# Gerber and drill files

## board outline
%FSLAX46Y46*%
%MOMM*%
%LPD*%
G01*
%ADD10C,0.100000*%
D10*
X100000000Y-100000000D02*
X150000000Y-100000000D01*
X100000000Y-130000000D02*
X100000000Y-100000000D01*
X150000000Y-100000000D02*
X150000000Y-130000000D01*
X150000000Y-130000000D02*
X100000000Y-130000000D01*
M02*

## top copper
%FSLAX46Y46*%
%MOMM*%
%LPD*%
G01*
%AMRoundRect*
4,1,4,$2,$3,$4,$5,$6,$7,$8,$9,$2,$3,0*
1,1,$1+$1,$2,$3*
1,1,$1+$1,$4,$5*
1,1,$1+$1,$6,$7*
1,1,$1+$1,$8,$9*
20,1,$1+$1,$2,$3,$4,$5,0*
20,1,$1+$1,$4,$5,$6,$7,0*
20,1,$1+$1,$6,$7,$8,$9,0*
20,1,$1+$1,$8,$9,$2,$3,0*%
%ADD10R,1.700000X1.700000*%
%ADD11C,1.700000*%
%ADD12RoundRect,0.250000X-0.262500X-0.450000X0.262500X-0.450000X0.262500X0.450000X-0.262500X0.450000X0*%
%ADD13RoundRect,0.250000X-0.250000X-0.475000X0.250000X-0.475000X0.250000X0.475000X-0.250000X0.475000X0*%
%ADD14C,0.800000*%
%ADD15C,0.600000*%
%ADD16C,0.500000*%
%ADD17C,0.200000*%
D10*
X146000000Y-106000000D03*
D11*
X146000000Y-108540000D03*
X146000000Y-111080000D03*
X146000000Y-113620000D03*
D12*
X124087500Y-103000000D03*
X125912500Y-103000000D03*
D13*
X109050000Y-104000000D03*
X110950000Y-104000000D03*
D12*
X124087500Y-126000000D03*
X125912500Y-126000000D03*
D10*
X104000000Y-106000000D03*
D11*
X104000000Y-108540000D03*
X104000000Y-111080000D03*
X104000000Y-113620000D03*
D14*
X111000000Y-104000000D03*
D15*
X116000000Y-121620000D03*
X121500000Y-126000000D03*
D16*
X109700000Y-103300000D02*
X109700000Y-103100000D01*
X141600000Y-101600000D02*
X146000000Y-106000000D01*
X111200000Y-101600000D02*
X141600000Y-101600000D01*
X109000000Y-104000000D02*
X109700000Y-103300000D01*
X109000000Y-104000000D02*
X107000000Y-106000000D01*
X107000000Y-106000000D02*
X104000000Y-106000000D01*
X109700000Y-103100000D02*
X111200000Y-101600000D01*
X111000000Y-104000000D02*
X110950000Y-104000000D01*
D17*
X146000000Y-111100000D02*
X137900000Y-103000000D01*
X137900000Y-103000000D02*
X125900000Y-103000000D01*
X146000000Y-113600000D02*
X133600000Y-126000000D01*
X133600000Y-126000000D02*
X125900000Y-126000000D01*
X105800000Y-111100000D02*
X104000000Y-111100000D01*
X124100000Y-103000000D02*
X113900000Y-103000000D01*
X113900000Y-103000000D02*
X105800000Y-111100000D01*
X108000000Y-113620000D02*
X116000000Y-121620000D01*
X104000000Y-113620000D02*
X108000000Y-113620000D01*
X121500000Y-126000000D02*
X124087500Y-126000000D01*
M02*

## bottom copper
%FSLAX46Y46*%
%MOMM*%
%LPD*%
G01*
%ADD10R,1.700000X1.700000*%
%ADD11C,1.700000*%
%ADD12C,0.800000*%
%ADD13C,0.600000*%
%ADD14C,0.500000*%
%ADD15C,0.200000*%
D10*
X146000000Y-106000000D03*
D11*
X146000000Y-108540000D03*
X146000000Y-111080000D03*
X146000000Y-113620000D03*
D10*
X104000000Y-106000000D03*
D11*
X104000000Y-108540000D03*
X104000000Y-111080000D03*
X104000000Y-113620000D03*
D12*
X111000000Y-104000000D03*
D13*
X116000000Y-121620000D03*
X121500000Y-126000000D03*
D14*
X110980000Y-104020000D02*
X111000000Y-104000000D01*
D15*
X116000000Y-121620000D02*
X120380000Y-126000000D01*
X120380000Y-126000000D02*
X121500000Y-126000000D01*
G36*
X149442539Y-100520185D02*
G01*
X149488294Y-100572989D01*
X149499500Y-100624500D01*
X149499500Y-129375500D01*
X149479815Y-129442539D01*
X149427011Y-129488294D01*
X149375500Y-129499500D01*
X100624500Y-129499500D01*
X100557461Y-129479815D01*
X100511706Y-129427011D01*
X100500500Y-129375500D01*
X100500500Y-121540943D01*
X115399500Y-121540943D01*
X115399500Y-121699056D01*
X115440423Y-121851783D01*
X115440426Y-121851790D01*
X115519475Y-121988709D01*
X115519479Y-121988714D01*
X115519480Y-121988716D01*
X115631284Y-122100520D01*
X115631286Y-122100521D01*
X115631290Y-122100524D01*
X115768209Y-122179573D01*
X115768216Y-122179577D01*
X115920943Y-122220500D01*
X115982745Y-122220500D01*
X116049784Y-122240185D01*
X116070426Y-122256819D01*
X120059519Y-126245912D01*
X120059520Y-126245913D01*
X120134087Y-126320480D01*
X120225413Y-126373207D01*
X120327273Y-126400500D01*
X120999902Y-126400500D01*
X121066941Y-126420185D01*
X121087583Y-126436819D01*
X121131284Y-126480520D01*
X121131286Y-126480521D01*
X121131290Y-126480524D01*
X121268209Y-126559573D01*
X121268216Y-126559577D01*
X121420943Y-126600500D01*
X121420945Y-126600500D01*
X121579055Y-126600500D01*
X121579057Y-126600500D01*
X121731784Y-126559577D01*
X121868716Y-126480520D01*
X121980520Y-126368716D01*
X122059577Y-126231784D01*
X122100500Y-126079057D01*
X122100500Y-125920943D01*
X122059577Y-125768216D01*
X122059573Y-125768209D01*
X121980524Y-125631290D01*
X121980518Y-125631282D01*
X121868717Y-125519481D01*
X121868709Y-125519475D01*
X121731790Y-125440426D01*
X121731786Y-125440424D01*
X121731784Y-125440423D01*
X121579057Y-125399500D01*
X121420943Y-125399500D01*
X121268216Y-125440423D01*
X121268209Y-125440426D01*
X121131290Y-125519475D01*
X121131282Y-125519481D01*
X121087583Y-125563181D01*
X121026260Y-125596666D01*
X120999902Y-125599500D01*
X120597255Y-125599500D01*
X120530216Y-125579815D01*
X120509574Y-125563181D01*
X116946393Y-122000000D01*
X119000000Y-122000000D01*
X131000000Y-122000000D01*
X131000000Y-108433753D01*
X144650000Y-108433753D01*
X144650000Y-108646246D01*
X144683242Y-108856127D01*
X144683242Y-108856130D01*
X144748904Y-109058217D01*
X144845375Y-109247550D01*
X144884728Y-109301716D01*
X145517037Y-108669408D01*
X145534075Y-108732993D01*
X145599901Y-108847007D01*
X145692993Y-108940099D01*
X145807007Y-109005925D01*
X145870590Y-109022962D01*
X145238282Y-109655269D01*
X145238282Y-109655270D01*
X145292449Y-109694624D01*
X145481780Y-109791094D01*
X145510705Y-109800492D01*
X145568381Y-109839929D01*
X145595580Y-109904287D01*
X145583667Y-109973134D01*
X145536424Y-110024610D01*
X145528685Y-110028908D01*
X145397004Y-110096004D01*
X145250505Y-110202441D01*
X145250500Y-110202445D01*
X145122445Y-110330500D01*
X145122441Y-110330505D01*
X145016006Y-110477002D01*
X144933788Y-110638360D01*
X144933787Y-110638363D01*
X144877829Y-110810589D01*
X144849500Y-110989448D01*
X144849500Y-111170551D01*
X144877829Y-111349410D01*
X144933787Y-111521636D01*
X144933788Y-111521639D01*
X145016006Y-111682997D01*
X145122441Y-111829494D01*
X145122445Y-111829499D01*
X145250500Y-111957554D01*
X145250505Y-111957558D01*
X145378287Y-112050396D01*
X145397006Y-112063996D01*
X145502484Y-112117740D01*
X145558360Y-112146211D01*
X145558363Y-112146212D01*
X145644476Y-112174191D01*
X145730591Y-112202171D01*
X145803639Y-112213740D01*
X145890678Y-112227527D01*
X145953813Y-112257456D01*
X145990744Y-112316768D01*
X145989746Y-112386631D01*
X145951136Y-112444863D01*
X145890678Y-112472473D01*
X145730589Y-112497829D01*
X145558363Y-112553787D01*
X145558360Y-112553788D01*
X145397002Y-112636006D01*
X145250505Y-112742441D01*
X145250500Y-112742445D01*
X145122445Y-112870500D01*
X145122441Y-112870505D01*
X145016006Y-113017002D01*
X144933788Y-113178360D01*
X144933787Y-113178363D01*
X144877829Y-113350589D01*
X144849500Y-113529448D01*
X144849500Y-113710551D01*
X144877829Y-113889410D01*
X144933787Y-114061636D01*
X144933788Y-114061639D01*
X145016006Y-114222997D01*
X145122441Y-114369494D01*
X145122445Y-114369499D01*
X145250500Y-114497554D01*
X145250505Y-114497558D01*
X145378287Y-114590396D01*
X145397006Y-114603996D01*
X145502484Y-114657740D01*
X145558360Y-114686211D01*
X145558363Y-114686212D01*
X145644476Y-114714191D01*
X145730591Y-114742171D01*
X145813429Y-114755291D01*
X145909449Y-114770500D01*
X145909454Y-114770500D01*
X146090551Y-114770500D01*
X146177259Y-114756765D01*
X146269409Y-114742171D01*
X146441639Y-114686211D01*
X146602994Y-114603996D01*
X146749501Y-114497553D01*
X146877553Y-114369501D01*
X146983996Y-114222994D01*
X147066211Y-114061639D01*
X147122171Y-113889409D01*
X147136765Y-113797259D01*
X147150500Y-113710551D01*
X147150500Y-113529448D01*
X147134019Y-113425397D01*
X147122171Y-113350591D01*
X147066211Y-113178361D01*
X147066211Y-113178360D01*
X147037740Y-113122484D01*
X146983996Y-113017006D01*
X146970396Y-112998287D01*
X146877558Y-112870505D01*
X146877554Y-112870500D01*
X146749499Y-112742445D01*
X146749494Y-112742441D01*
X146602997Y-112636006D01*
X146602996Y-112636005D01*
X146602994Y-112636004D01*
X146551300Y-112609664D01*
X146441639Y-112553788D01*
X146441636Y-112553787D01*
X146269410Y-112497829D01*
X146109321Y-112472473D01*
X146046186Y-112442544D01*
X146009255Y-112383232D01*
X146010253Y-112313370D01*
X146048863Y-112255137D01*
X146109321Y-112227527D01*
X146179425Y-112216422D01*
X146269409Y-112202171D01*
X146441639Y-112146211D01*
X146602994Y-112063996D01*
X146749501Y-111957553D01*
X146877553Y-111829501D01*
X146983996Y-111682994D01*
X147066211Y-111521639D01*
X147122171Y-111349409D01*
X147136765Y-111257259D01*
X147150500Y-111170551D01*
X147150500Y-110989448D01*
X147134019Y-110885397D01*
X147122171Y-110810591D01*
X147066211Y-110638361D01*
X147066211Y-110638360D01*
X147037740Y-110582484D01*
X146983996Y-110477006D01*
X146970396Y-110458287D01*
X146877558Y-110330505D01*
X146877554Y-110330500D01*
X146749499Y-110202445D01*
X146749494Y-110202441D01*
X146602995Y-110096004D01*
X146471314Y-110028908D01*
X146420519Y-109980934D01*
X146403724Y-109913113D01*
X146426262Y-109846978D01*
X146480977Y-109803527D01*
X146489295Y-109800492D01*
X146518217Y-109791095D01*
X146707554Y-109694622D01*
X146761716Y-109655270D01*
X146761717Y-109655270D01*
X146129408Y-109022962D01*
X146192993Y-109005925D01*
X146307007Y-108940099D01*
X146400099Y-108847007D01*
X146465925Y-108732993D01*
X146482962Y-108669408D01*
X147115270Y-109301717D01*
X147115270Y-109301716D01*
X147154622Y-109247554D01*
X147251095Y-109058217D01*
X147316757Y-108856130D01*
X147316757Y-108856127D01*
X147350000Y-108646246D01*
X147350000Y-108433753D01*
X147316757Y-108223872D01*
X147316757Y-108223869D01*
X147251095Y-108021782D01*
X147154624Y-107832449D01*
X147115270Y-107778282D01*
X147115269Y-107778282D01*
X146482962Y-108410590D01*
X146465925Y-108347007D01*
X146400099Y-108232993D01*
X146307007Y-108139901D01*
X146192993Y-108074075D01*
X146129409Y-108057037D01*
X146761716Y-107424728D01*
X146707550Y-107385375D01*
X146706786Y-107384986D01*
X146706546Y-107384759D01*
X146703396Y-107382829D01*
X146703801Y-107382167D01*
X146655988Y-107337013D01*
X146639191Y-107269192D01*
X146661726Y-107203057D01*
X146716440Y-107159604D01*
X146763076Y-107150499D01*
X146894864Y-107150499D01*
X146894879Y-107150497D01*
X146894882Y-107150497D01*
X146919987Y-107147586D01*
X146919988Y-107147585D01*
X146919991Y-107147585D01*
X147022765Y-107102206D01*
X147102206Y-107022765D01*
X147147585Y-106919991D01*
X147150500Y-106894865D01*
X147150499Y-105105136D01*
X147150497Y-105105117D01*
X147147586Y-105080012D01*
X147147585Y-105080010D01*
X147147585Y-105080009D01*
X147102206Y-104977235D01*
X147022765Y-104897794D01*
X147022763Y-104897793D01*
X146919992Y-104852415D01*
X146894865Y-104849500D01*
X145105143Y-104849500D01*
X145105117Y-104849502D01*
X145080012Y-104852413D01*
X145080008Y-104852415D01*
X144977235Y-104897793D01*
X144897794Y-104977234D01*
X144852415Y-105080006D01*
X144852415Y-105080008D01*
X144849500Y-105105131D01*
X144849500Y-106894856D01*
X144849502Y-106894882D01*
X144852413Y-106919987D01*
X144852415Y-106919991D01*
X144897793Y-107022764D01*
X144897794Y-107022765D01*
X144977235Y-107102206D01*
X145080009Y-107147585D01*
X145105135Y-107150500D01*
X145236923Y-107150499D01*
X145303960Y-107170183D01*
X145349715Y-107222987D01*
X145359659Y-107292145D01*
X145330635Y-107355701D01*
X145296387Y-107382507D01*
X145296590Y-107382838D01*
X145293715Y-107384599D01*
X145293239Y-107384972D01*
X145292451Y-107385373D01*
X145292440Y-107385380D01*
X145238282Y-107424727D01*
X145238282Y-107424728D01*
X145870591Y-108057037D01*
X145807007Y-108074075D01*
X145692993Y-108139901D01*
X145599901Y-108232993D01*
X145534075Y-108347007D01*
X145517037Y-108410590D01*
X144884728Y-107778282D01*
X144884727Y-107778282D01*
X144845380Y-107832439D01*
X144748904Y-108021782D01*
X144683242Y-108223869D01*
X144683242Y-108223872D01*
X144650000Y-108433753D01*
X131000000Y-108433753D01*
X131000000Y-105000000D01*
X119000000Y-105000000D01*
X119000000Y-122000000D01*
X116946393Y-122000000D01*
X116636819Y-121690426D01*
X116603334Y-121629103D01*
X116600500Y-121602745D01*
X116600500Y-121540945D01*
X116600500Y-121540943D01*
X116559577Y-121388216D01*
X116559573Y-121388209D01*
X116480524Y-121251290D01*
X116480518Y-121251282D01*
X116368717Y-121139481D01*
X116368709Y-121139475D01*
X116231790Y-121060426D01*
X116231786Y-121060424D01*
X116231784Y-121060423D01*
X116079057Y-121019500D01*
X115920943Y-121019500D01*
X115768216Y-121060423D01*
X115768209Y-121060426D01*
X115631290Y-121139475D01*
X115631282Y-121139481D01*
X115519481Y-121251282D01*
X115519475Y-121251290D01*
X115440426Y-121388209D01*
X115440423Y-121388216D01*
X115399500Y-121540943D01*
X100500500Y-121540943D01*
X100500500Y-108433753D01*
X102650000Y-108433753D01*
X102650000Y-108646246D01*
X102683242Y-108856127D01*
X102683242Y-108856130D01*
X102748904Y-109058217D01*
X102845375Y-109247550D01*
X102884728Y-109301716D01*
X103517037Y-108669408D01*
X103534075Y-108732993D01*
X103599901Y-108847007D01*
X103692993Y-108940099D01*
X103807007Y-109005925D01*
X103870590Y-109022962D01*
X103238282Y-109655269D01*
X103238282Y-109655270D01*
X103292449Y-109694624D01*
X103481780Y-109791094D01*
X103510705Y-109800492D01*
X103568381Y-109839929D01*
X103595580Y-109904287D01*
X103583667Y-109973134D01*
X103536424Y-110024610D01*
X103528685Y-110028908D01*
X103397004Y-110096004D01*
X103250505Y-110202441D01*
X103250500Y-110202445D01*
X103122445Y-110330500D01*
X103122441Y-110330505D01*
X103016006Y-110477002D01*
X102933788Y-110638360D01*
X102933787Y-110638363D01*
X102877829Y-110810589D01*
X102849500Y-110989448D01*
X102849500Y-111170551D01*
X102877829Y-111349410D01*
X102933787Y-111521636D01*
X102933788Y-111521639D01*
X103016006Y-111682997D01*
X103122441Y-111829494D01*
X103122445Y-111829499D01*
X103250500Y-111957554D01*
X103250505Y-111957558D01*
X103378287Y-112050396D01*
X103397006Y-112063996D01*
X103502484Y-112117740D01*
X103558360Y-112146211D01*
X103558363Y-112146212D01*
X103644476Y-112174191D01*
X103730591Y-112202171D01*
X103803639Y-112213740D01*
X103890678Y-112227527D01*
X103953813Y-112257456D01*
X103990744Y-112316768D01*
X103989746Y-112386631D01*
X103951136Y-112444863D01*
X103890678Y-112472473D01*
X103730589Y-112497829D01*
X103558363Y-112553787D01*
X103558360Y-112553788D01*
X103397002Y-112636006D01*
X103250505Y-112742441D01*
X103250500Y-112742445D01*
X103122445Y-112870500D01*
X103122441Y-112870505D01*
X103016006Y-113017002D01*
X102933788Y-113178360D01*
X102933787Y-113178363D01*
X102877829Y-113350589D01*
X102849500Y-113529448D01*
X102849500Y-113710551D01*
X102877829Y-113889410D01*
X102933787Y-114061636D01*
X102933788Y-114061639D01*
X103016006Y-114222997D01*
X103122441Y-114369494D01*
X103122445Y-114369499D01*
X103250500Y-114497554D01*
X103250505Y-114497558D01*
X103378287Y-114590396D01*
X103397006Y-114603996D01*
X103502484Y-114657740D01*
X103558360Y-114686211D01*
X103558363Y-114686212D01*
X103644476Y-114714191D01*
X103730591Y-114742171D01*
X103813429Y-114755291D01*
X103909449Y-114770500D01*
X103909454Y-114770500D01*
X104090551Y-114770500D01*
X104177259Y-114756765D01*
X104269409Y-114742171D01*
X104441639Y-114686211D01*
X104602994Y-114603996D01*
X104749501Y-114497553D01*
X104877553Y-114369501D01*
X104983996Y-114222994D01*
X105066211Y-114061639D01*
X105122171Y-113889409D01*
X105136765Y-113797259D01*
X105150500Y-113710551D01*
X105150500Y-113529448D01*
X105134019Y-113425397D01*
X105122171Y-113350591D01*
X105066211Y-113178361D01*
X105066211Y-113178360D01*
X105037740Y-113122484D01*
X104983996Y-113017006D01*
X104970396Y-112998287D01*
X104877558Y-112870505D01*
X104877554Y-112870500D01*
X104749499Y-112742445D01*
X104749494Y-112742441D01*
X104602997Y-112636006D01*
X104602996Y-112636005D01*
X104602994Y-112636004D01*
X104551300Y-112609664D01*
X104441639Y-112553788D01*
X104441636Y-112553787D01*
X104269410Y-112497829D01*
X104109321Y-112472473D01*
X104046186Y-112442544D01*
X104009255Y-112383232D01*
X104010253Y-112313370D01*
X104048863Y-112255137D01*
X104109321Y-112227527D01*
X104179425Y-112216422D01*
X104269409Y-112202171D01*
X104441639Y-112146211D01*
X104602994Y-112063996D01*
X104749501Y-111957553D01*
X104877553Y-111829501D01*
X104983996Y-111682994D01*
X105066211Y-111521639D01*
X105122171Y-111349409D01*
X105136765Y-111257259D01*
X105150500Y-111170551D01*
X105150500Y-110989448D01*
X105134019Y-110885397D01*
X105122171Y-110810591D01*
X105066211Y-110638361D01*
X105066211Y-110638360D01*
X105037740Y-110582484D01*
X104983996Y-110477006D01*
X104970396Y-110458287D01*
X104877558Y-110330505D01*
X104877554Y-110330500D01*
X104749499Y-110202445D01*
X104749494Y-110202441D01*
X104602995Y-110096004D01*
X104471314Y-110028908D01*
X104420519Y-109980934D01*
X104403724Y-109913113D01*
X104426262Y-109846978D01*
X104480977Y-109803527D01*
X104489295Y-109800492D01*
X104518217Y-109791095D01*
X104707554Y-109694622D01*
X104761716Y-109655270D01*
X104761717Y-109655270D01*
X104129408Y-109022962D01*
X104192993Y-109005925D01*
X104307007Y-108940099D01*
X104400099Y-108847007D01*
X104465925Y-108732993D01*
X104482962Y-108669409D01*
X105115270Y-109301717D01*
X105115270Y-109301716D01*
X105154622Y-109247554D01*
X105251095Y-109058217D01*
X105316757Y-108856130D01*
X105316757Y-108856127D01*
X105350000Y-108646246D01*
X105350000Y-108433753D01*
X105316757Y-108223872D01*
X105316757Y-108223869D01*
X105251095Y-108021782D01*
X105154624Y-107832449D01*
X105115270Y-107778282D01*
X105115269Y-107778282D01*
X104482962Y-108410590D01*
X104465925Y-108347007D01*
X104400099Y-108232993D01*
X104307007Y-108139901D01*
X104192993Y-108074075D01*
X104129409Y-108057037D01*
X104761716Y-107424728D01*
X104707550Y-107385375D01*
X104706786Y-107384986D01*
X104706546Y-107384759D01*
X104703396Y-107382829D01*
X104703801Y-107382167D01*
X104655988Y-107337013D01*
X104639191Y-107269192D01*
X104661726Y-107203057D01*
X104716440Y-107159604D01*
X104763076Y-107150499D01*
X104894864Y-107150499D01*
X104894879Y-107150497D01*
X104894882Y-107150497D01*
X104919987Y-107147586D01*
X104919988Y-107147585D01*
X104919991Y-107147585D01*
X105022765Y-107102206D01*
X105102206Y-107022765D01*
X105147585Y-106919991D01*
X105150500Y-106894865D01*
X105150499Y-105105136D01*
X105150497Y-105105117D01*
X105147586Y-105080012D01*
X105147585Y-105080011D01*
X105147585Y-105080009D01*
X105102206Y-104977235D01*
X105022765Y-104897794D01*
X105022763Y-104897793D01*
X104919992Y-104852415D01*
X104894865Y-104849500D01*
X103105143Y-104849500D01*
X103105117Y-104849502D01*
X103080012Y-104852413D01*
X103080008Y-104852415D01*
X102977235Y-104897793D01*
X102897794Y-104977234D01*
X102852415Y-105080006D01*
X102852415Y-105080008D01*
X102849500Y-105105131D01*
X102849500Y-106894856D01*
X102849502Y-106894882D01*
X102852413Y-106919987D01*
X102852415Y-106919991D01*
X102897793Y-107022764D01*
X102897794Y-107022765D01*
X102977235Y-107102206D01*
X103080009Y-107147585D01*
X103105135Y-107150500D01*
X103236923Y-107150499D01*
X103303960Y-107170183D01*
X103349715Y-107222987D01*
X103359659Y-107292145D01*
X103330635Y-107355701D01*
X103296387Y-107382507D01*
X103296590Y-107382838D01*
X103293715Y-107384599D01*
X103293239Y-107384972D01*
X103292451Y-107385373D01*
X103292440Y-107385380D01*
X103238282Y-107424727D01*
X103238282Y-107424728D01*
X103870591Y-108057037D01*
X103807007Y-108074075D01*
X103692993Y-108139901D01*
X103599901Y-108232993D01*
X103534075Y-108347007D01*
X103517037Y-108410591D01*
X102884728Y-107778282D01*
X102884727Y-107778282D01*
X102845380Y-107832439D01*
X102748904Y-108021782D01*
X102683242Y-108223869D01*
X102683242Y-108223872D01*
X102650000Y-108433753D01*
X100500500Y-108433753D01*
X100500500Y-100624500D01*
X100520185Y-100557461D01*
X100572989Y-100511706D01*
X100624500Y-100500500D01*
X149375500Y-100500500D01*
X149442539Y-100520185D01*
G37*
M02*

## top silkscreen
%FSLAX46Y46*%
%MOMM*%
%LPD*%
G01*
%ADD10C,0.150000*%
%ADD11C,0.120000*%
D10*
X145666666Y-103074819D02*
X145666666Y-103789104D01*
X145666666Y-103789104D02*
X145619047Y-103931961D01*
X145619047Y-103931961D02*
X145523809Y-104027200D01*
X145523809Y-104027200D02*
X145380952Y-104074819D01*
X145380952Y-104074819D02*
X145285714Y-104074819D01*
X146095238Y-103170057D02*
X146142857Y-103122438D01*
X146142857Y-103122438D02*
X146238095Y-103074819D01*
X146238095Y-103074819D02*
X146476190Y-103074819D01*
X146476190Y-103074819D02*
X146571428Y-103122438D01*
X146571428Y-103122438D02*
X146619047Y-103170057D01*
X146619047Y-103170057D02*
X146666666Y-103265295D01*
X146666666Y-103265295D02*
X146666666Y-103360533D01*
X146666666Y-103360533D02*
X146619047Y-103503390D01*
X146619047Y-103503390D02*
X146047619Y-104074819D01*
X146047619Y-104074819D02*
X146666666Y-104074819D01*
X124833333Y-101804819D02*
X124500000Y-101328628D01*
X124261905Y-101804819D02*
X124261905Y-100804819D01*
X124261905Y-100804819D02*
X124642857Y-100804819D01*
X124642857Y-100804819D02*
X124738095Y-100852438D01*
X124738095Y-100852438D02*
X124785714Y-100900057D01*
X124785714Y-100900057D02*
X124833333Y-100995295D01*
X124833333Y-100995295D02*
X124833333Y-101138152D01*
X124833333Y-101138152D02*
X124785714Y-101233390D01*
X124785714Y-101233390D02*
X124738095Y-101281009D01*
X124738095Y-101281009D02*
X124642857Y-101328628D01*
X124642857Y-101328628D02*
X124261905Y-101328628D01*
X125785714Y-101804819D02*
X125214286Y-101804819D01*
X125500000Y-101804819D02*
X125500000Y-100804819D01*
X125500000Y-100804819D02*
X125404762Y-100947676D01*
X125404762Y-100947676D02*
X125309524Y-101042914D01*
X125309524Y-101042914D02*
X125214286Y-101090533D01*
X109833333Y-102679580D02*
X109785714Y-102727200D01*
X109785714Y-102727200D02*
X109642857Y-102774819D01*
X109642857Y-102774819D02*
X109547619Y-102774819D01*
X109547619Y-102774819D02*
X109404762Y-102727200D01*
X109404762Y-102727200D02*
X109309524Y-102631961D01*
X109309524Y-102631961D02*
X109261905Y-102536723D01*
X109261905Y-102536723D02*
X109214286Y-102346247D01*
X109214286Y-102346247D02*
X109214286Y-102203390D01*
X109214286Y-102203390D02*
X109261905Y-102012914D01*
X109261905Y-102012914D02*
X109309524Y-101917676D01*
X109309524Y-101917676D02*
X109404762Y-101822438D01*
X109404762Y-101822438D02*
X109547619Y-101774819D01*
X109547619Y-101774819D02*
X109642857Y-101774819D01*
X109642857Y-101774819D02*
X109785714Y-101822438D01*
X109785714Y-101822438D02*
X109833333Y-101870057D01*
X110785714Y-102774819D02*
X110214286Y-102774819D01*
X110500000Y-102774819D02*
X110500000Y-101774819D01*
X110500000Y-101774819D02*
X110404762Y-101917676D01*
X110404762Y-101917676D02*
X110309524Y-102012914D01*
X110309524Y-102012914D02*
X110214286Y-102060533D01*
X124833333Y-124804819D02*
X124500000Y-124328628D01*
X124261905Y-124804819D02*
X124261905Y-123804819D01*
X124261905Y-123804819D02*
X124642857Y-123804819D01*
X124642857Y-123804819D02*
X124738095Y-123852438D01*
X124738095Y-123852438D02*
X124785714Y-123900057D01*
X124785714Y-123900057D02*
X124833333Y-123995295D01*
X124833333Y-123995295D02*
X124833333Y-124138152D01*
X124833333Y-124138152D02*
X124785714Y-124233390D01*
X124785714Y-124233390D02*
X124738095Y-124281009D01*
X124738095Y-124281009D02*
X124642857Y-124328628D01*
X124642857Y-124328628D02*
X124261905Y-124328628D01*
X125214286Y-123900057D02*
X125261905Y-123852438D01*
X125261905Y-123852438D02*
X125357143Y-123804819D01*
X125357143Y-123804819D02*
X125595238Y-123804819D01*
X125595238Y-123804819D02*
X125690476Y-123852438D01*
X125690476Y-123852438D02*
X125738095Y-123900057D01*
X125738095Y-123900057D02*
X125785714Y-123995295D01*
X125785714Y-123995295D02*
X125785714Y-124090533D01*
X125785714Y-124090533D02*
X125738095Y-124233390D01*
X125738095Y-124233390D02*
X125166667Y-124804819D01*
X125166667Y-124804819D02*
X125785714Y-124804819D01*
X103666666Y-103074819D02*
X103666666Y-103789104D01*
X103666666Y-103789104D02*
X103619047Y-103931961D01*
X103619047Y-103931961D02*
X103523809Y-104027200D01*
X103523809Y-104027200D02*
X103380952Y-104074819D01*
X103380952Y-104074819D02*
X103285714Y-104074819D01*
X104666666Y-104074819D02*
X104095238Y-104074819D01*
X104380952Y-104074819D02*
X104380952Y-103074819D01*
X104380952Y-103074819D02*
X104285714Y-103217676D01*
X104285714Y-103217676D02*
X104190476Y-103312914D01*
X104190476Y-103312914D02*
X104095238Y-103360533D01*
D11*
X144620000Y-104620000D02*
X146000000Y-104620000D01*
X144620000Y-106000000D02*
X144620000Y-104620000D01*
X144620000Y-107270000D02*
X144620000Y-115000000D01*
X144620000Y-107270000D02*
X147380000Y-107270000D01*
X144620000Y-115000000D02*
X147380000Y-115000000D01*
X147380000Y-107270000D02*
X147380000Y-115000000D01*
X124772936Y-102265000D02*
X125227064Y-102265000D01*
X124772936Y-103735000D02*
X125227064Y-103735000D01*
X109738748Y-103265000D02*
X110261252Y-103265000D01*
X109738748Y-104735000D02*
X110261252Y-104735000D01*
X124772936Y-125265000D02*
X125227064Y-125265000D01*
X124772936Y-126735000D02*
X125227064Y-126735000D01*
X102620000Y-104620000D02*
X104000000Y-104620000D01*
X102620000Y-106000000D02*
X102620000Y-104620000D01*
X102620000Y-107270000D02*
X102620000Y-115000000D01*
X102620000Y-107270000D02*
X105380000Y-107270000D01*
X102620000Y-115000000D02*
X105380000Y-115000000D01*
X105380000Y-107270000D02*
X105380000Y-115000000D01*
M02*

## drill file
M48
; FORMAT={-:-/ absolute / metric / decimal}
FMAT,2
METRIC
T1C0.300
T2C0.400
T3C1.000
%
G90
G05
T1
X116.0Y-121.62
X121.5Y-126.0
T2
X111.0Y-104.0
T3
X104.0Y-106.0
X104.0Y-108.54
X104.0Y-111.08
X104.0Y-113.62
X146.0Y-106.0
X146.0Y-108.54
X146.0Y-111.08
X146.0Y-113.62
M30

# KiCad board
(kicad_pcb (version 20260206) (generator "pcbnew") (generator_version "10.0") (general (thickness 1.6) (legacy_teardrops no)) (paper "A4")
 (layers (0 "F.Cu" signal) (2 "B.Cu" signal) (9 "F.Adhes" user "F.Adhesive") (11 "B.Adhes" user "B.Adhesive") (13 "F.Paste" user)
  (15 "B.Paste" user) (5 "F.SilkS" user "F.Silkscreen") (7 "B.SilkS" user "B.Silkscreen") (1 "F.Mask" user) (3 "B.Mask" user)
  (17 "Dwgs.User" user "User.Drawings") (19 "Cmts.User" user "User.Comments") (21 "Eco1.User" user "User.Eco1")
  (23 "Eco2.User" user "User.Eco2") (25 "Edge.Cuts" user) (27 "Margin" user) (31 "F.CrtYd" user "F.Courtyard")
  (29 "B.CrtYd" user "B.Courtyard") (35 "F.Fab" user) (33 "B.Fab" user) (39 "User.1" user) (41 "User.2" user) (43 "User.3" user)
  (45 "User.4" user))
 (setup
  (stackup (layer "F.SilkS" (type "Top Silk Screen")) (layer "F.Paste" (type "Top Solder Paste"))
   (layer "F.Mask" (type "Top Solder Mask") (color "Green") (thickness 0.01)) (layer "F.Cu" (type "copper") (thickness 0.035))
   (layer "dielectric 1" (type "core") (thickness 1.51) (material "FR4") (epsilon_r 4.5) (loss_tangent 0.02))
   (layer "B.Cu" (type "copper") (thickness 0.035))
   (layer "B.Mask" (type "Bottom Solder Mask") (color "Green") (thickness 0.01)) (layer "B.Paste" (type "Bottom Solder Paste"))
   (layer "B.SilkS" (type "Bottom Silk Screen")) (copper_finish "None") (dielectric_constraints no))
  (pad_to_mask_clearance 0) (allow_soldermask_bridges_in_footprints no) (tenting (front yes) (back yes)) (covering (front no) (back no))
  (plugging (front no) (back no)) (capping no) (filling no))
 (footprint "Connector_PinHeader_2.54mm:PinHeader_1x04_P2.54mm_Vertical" (layer "F.Cu") (at 146 106)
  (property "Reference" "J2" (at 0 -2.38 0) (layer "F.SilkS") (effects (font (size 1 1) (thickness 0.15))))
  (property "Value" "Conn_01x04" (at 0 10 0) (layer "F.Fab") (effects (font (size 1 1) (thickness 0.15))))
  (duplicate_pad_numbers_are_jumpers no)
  (fp_line (start -1.38 -1.38) (end 0 -1.38) (stroke (width 0.12) (type solid)) (layer "F.SilkS"))
  (fp_line (start -1.38 0) (end -1.38 -1.38) (stroke (width 0.12) (type solid)) (layer "F.SilkS"))
  (fp_line (start -1.38 1.27) (end -1.38 9) (stroke (width 0.12) (type solid)) (layer "F.SilkS"))
  (fp_line (start -1.38 1.27) (end 1.38 1.27) (stroke (width 0.12) (type solid)) (layer "F.SilkS"))
  (fp_line (start -1.38 9) (end 1.38 9) (stroke (width 0.12) (type solid)) (layer "F.SilkS"))
  (fp_line (start 1.38 1.27) (end 1.38 9) (stroke (width 0.12) (type solid)) (layer "F.SilkS"))
  (pad "1" thru_hole rect (at 0 0) (size 1.7 1.7) (drill 1) (layers "*.Cu" "*.Mask") (remove_unused_layers no) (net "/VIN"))
  (pad "2" thru_hole circle (at 0 2.54) (size 1.7 1.7) (drill 1) (layers "*.Cu" "*.Mask") (remove_unused_layers no) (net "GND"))
  (pad "3" thru_hole circle (at 0 5.08) (size 1.7 1.7) (drill 1) (layers "*.Cu" "*.Mask") (remove_unused_layers no) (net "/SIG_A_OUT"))
  (pad "4" thru_hole circle (at 0 7.62) (size 1.7 1.7) (drill 1) (layers "*.Cu" "*.Mask") (remove_unused_layers no) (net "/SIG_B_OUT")))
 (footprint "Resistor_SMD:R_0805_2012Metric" (layer "F.Cu") (at 125 103)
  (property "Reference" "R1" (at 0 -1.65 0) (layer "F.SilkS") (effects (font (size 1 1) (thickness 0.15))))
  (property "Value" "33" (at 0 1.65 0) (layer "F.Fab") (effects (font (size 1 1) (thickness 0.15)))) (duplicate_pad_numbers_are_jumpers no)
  (fp_line (start -0.227064 -0.735) (end 0.227064 -0.735) (stroke (width 0.12) (type solid)) (layer "F.SilkS"))
  (fp_line (start -0.227064 0.735) (end 0.227064 0.735) (stroke (width 0.12) (type solid)) (layer "F.SilkS"))
  (pad "1" smd roundrect (at -0.9125 0) (size 1.025 1.4) (layers "F.Cu" "F.Mask" "F.Paste") (roundrect_rratio 0.243902) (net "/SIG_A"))
  (pad "2" smd roundrect (at 0.9125 0) (size 1.025 1.4) (layers "F.Cu" "F.Mask" "F.Paste") (roundrect_rratio 0.243902) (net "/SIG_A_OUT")))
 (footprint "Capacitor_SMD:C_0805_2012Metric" (layer "F.Cu") (at 110 104)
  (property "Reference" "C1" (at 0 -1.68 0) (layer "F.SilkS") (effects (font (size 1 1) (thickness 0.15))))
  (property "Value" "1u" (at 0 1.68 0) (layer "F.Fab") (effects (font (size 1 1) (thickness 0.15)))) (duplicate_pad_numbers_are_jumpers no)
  (fp_line (start -0.261252 -0.735) (end 0.261252 -0.735) (stroke (width 0.12) (type solid)) (layer "F.SilkS"))
  (fp_line (start -0.261252 0.735) (end 0.261252 0.735) (stroke (width 0.12) (type solid)) (layer "F.SilkS"))
  (pad "1" smd roundrect (at -0.95 0) (size 1 1.45) (layers "F.Cu" "F.Mask" "F.Paste") (roundrect_rratio 0.25) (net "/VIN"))
  (pad "2" smd roundrect (at 0.95 0) (size 1 1.45) (layers "F.Cu" "F.Mask" "F.Paste") (roundrect_rratio 0.25) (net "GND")))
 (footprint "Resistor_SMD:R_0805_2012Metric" (layer "F.Cu") (at 125 126)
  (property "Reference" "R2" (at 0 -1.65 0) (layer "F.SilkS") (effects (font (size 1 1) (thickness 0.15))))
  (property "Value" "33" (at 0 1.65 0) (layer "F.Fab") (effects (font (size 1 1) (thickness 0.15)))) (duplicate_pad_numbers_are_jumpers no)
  (fp_line (start -0.227064 -0.735) (end 0.227064 -0.735) (stroke (width 0.12) (type solid)) (layer "F.SilkS"))
  (fp_line (start -0.227064 0.735) (end 0.227064 0.735) (stroke (width 0.12) (type solid)) (layer "F.SilkS"))
  (pad "1" smd roundrect (at -0.9125 0) (size 1.025 1.4) (layers "F.Cu" "F.Mask" "F.Paste") (roundrect_rratio 0.243902) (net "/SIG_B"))
  (pad "2" smd roundrect (at 0.9125 0) (size 1.025 1.4) (layers "F.Cu" "F.Mask" "F.Paste") (roundrect_rratio 0.243902) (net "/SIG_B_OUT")))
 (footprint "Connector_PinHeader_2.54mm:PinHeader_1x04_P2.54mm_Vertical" (layer "F.Cu") (at 104 106)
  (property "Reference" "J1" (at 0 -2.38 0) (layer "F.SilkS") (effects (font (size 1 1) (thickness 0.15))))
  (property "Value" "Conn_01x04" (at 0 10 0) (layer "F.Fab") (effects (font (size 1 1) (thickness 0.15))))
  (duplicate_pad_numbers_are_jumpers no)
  (fp_line (start -1.38 -1.38) (end 0 -1.38) (stroke (width 0.12) (type solid)) (layer "F.SilkS"))
  (fp_line (start -1.38 0) (end -1.38 -1.38) (stroke (width 0.12) (type solid)) (layer "F.SilkS"))
  (fp_line (start -1.38 1.27) (end -1.38 9) (stroke (width 0.12) (type solid)) (layer "F.SilkS"))
  (fp_line (start -1.38 1.27) (end 1.38 1.27) (stroke (width 0.12) (type solid)) (layer "F.SilkS"))
  (fp_line (start -1.38 9) (end 1.38 9) (stroke (width 0.12) (type solid)) (layer "F.SilkS"))
  (fp_line (start 1.38 1.27) (end 1.38 9) (stroke (width 0.12) (type solid)) (layer "F.SilkS"))
  (pad "1" thru_hole rect (at 0 0) (size 1.7 1.7) (drill 1) (layers "*.Cu" "*.Mask") (remove_unused_layers no) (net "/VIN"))
  (pad "2" thru_hole circle (at 0 2.54) (size 1.7 1.7) (drill 1) (layers "*.Cu" "*.Mask") (remove_unused_layers no) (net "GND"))
  (pad "3" thru_hole circle (at 0 5.08) (size 1.7 1.7) (drill 1) (layers "*.Cu" "*.Mask") (remove_unused_layers no) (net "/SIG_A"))
  (pad "4" thru_hole circle (at 0 7.62) (size 1.7 1.7) (drill 1) (layers "*.Cu" "*.Mask") (remove_unused_layers no) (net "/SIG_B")))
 (gr_line (start 100 100) (end 150 100) (stroke (width 0.1) (type default)) (layer "Edge.Cuts"))
 (gr_line (start 100 130) (end 100 100) (stroke (width 0.1) (type default)) (layer "Edge.Cuts"))
 (gr_line (start 150 100) (end 150 130) (stroke (width 0.1) (type default)) (layer "Edge.Cuts"))
 (gr_line (start 150 130) (end 100 130) (stroke (width 0.1) (type default)) (layer "Edge.Cuts"))
 (segment (start 109.7 103.3) (end 109.7 103.1) (width 0.5) (layer "F.Cu") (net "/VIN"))
 (segment (start 141.6 101.6) (end 146 106) (width 0.5) (layer "F.Cu") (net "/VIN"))
 (segment (start 111.2 101.6) (end 141.6 101.6) (width 0.5) (layer "F.Cu") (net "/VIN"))
 (segment (start 109 104) (end 109.7 103.3) (width 0.5) (layer "F.Cu") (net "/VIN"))
 (segment (start 109 104) (end 107 106) (width 0.5) (layer "F.Cu") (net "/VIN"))
 (segment (start 107 106) (end 104 106) (width 0.5) (layer "F.Cu") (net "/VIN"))
 (segment (start 109.7 103.1) (end 111.2 101.6) (width 0.5) (layer "F.Cu") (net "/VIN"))
 (segment (start 111 104) (end 110.95 104) (width 0.5) (layer "F.Cu") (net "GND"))
 (via (at 111 104) (size 0.8) (drill 0.4) (layers "F.Cu" "B.Cu") (capping yes) (filling yes) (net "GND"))
 (segment (start 110.98 104.02) (end 111 104) (width 0.5) (layer "B.Cu") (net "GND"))
 (segment (start 146 111.1) (end 137.9 103) (width 0.2) (layer "F.Cu") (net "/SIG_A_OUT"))
 (segment (start 137.9 103) (end 125.9 103) (width 0.2) (layer "F.Cu") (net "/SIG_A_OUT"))
 (segment (start 146 113.6) (end 133.6 126) (width 0.2) (layer "F.Cu") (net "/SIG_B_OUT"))
 (segment (start 133.6 126) (end 125.9 126) (width 0.2) (layer "F.Cu") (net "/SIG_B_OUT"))
 (segment (start 105.8 111.1) (end 104 111.1) (width 0.2) (layer "F.Cu") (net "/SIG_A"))
 (segment (start 124.1 103) (end 113.9 103) (width 0.2) (layer "F.Cu") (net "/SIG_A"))
 (segment (start 113.9 103) (end 105.8 111.1) (width 0.2) (layer "F.Cu") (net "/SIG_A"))
 (segment (start 108 113.62) (end 116 121.62) (width 0.2) (locked yes) (layer "F.Cu") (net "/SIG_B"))
 (segment (start 104 113.62) (end 108 113.62) (width 0.2) (locked yes) (layer "F.Cu") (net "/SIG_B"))
 (segment (start 121.5 126) (end 124.0875 126) (width 0.2) (locked yes) (layer "F.Cu") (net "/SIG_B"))
 (via (at 116 121.62) (size 0.6) (drill 0.3) (layers "F.Cu" "B.Cu") (locked yes) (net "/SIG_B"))
 (via (at 121.5 126) (size 0.6) (drill 0.3) (layers "F.Cu" "B.Cu") (locked yes) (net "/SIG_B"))
 (segment (start 116 121.62) (end 120.38 126) (width 0.2) (locked yes) (layer "B.Cu") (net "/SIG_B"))
 (segment (start 120.38 126) (end 121.5 126) (width 0.2) (locked yes) (layer "B.Cu") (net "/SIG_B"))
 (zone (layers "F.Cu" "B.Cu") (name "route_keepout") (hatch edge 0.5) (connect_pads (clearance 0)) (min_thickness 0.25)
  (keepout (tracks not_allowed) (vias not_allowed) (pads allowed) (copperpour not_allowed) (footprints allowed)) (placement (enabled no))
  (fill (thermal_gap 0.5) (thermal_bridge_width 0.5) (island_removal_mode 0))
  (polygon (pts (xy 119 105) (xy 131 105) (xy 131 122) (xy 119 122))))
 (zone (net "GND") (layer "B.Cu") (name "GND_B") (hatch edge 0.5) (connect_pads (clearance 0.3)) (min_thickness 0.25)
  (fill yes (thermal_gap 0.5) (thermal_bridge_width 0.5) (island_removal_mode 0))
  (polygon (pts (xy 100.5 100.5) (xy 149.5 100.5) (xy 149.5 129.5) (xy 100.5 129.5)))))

